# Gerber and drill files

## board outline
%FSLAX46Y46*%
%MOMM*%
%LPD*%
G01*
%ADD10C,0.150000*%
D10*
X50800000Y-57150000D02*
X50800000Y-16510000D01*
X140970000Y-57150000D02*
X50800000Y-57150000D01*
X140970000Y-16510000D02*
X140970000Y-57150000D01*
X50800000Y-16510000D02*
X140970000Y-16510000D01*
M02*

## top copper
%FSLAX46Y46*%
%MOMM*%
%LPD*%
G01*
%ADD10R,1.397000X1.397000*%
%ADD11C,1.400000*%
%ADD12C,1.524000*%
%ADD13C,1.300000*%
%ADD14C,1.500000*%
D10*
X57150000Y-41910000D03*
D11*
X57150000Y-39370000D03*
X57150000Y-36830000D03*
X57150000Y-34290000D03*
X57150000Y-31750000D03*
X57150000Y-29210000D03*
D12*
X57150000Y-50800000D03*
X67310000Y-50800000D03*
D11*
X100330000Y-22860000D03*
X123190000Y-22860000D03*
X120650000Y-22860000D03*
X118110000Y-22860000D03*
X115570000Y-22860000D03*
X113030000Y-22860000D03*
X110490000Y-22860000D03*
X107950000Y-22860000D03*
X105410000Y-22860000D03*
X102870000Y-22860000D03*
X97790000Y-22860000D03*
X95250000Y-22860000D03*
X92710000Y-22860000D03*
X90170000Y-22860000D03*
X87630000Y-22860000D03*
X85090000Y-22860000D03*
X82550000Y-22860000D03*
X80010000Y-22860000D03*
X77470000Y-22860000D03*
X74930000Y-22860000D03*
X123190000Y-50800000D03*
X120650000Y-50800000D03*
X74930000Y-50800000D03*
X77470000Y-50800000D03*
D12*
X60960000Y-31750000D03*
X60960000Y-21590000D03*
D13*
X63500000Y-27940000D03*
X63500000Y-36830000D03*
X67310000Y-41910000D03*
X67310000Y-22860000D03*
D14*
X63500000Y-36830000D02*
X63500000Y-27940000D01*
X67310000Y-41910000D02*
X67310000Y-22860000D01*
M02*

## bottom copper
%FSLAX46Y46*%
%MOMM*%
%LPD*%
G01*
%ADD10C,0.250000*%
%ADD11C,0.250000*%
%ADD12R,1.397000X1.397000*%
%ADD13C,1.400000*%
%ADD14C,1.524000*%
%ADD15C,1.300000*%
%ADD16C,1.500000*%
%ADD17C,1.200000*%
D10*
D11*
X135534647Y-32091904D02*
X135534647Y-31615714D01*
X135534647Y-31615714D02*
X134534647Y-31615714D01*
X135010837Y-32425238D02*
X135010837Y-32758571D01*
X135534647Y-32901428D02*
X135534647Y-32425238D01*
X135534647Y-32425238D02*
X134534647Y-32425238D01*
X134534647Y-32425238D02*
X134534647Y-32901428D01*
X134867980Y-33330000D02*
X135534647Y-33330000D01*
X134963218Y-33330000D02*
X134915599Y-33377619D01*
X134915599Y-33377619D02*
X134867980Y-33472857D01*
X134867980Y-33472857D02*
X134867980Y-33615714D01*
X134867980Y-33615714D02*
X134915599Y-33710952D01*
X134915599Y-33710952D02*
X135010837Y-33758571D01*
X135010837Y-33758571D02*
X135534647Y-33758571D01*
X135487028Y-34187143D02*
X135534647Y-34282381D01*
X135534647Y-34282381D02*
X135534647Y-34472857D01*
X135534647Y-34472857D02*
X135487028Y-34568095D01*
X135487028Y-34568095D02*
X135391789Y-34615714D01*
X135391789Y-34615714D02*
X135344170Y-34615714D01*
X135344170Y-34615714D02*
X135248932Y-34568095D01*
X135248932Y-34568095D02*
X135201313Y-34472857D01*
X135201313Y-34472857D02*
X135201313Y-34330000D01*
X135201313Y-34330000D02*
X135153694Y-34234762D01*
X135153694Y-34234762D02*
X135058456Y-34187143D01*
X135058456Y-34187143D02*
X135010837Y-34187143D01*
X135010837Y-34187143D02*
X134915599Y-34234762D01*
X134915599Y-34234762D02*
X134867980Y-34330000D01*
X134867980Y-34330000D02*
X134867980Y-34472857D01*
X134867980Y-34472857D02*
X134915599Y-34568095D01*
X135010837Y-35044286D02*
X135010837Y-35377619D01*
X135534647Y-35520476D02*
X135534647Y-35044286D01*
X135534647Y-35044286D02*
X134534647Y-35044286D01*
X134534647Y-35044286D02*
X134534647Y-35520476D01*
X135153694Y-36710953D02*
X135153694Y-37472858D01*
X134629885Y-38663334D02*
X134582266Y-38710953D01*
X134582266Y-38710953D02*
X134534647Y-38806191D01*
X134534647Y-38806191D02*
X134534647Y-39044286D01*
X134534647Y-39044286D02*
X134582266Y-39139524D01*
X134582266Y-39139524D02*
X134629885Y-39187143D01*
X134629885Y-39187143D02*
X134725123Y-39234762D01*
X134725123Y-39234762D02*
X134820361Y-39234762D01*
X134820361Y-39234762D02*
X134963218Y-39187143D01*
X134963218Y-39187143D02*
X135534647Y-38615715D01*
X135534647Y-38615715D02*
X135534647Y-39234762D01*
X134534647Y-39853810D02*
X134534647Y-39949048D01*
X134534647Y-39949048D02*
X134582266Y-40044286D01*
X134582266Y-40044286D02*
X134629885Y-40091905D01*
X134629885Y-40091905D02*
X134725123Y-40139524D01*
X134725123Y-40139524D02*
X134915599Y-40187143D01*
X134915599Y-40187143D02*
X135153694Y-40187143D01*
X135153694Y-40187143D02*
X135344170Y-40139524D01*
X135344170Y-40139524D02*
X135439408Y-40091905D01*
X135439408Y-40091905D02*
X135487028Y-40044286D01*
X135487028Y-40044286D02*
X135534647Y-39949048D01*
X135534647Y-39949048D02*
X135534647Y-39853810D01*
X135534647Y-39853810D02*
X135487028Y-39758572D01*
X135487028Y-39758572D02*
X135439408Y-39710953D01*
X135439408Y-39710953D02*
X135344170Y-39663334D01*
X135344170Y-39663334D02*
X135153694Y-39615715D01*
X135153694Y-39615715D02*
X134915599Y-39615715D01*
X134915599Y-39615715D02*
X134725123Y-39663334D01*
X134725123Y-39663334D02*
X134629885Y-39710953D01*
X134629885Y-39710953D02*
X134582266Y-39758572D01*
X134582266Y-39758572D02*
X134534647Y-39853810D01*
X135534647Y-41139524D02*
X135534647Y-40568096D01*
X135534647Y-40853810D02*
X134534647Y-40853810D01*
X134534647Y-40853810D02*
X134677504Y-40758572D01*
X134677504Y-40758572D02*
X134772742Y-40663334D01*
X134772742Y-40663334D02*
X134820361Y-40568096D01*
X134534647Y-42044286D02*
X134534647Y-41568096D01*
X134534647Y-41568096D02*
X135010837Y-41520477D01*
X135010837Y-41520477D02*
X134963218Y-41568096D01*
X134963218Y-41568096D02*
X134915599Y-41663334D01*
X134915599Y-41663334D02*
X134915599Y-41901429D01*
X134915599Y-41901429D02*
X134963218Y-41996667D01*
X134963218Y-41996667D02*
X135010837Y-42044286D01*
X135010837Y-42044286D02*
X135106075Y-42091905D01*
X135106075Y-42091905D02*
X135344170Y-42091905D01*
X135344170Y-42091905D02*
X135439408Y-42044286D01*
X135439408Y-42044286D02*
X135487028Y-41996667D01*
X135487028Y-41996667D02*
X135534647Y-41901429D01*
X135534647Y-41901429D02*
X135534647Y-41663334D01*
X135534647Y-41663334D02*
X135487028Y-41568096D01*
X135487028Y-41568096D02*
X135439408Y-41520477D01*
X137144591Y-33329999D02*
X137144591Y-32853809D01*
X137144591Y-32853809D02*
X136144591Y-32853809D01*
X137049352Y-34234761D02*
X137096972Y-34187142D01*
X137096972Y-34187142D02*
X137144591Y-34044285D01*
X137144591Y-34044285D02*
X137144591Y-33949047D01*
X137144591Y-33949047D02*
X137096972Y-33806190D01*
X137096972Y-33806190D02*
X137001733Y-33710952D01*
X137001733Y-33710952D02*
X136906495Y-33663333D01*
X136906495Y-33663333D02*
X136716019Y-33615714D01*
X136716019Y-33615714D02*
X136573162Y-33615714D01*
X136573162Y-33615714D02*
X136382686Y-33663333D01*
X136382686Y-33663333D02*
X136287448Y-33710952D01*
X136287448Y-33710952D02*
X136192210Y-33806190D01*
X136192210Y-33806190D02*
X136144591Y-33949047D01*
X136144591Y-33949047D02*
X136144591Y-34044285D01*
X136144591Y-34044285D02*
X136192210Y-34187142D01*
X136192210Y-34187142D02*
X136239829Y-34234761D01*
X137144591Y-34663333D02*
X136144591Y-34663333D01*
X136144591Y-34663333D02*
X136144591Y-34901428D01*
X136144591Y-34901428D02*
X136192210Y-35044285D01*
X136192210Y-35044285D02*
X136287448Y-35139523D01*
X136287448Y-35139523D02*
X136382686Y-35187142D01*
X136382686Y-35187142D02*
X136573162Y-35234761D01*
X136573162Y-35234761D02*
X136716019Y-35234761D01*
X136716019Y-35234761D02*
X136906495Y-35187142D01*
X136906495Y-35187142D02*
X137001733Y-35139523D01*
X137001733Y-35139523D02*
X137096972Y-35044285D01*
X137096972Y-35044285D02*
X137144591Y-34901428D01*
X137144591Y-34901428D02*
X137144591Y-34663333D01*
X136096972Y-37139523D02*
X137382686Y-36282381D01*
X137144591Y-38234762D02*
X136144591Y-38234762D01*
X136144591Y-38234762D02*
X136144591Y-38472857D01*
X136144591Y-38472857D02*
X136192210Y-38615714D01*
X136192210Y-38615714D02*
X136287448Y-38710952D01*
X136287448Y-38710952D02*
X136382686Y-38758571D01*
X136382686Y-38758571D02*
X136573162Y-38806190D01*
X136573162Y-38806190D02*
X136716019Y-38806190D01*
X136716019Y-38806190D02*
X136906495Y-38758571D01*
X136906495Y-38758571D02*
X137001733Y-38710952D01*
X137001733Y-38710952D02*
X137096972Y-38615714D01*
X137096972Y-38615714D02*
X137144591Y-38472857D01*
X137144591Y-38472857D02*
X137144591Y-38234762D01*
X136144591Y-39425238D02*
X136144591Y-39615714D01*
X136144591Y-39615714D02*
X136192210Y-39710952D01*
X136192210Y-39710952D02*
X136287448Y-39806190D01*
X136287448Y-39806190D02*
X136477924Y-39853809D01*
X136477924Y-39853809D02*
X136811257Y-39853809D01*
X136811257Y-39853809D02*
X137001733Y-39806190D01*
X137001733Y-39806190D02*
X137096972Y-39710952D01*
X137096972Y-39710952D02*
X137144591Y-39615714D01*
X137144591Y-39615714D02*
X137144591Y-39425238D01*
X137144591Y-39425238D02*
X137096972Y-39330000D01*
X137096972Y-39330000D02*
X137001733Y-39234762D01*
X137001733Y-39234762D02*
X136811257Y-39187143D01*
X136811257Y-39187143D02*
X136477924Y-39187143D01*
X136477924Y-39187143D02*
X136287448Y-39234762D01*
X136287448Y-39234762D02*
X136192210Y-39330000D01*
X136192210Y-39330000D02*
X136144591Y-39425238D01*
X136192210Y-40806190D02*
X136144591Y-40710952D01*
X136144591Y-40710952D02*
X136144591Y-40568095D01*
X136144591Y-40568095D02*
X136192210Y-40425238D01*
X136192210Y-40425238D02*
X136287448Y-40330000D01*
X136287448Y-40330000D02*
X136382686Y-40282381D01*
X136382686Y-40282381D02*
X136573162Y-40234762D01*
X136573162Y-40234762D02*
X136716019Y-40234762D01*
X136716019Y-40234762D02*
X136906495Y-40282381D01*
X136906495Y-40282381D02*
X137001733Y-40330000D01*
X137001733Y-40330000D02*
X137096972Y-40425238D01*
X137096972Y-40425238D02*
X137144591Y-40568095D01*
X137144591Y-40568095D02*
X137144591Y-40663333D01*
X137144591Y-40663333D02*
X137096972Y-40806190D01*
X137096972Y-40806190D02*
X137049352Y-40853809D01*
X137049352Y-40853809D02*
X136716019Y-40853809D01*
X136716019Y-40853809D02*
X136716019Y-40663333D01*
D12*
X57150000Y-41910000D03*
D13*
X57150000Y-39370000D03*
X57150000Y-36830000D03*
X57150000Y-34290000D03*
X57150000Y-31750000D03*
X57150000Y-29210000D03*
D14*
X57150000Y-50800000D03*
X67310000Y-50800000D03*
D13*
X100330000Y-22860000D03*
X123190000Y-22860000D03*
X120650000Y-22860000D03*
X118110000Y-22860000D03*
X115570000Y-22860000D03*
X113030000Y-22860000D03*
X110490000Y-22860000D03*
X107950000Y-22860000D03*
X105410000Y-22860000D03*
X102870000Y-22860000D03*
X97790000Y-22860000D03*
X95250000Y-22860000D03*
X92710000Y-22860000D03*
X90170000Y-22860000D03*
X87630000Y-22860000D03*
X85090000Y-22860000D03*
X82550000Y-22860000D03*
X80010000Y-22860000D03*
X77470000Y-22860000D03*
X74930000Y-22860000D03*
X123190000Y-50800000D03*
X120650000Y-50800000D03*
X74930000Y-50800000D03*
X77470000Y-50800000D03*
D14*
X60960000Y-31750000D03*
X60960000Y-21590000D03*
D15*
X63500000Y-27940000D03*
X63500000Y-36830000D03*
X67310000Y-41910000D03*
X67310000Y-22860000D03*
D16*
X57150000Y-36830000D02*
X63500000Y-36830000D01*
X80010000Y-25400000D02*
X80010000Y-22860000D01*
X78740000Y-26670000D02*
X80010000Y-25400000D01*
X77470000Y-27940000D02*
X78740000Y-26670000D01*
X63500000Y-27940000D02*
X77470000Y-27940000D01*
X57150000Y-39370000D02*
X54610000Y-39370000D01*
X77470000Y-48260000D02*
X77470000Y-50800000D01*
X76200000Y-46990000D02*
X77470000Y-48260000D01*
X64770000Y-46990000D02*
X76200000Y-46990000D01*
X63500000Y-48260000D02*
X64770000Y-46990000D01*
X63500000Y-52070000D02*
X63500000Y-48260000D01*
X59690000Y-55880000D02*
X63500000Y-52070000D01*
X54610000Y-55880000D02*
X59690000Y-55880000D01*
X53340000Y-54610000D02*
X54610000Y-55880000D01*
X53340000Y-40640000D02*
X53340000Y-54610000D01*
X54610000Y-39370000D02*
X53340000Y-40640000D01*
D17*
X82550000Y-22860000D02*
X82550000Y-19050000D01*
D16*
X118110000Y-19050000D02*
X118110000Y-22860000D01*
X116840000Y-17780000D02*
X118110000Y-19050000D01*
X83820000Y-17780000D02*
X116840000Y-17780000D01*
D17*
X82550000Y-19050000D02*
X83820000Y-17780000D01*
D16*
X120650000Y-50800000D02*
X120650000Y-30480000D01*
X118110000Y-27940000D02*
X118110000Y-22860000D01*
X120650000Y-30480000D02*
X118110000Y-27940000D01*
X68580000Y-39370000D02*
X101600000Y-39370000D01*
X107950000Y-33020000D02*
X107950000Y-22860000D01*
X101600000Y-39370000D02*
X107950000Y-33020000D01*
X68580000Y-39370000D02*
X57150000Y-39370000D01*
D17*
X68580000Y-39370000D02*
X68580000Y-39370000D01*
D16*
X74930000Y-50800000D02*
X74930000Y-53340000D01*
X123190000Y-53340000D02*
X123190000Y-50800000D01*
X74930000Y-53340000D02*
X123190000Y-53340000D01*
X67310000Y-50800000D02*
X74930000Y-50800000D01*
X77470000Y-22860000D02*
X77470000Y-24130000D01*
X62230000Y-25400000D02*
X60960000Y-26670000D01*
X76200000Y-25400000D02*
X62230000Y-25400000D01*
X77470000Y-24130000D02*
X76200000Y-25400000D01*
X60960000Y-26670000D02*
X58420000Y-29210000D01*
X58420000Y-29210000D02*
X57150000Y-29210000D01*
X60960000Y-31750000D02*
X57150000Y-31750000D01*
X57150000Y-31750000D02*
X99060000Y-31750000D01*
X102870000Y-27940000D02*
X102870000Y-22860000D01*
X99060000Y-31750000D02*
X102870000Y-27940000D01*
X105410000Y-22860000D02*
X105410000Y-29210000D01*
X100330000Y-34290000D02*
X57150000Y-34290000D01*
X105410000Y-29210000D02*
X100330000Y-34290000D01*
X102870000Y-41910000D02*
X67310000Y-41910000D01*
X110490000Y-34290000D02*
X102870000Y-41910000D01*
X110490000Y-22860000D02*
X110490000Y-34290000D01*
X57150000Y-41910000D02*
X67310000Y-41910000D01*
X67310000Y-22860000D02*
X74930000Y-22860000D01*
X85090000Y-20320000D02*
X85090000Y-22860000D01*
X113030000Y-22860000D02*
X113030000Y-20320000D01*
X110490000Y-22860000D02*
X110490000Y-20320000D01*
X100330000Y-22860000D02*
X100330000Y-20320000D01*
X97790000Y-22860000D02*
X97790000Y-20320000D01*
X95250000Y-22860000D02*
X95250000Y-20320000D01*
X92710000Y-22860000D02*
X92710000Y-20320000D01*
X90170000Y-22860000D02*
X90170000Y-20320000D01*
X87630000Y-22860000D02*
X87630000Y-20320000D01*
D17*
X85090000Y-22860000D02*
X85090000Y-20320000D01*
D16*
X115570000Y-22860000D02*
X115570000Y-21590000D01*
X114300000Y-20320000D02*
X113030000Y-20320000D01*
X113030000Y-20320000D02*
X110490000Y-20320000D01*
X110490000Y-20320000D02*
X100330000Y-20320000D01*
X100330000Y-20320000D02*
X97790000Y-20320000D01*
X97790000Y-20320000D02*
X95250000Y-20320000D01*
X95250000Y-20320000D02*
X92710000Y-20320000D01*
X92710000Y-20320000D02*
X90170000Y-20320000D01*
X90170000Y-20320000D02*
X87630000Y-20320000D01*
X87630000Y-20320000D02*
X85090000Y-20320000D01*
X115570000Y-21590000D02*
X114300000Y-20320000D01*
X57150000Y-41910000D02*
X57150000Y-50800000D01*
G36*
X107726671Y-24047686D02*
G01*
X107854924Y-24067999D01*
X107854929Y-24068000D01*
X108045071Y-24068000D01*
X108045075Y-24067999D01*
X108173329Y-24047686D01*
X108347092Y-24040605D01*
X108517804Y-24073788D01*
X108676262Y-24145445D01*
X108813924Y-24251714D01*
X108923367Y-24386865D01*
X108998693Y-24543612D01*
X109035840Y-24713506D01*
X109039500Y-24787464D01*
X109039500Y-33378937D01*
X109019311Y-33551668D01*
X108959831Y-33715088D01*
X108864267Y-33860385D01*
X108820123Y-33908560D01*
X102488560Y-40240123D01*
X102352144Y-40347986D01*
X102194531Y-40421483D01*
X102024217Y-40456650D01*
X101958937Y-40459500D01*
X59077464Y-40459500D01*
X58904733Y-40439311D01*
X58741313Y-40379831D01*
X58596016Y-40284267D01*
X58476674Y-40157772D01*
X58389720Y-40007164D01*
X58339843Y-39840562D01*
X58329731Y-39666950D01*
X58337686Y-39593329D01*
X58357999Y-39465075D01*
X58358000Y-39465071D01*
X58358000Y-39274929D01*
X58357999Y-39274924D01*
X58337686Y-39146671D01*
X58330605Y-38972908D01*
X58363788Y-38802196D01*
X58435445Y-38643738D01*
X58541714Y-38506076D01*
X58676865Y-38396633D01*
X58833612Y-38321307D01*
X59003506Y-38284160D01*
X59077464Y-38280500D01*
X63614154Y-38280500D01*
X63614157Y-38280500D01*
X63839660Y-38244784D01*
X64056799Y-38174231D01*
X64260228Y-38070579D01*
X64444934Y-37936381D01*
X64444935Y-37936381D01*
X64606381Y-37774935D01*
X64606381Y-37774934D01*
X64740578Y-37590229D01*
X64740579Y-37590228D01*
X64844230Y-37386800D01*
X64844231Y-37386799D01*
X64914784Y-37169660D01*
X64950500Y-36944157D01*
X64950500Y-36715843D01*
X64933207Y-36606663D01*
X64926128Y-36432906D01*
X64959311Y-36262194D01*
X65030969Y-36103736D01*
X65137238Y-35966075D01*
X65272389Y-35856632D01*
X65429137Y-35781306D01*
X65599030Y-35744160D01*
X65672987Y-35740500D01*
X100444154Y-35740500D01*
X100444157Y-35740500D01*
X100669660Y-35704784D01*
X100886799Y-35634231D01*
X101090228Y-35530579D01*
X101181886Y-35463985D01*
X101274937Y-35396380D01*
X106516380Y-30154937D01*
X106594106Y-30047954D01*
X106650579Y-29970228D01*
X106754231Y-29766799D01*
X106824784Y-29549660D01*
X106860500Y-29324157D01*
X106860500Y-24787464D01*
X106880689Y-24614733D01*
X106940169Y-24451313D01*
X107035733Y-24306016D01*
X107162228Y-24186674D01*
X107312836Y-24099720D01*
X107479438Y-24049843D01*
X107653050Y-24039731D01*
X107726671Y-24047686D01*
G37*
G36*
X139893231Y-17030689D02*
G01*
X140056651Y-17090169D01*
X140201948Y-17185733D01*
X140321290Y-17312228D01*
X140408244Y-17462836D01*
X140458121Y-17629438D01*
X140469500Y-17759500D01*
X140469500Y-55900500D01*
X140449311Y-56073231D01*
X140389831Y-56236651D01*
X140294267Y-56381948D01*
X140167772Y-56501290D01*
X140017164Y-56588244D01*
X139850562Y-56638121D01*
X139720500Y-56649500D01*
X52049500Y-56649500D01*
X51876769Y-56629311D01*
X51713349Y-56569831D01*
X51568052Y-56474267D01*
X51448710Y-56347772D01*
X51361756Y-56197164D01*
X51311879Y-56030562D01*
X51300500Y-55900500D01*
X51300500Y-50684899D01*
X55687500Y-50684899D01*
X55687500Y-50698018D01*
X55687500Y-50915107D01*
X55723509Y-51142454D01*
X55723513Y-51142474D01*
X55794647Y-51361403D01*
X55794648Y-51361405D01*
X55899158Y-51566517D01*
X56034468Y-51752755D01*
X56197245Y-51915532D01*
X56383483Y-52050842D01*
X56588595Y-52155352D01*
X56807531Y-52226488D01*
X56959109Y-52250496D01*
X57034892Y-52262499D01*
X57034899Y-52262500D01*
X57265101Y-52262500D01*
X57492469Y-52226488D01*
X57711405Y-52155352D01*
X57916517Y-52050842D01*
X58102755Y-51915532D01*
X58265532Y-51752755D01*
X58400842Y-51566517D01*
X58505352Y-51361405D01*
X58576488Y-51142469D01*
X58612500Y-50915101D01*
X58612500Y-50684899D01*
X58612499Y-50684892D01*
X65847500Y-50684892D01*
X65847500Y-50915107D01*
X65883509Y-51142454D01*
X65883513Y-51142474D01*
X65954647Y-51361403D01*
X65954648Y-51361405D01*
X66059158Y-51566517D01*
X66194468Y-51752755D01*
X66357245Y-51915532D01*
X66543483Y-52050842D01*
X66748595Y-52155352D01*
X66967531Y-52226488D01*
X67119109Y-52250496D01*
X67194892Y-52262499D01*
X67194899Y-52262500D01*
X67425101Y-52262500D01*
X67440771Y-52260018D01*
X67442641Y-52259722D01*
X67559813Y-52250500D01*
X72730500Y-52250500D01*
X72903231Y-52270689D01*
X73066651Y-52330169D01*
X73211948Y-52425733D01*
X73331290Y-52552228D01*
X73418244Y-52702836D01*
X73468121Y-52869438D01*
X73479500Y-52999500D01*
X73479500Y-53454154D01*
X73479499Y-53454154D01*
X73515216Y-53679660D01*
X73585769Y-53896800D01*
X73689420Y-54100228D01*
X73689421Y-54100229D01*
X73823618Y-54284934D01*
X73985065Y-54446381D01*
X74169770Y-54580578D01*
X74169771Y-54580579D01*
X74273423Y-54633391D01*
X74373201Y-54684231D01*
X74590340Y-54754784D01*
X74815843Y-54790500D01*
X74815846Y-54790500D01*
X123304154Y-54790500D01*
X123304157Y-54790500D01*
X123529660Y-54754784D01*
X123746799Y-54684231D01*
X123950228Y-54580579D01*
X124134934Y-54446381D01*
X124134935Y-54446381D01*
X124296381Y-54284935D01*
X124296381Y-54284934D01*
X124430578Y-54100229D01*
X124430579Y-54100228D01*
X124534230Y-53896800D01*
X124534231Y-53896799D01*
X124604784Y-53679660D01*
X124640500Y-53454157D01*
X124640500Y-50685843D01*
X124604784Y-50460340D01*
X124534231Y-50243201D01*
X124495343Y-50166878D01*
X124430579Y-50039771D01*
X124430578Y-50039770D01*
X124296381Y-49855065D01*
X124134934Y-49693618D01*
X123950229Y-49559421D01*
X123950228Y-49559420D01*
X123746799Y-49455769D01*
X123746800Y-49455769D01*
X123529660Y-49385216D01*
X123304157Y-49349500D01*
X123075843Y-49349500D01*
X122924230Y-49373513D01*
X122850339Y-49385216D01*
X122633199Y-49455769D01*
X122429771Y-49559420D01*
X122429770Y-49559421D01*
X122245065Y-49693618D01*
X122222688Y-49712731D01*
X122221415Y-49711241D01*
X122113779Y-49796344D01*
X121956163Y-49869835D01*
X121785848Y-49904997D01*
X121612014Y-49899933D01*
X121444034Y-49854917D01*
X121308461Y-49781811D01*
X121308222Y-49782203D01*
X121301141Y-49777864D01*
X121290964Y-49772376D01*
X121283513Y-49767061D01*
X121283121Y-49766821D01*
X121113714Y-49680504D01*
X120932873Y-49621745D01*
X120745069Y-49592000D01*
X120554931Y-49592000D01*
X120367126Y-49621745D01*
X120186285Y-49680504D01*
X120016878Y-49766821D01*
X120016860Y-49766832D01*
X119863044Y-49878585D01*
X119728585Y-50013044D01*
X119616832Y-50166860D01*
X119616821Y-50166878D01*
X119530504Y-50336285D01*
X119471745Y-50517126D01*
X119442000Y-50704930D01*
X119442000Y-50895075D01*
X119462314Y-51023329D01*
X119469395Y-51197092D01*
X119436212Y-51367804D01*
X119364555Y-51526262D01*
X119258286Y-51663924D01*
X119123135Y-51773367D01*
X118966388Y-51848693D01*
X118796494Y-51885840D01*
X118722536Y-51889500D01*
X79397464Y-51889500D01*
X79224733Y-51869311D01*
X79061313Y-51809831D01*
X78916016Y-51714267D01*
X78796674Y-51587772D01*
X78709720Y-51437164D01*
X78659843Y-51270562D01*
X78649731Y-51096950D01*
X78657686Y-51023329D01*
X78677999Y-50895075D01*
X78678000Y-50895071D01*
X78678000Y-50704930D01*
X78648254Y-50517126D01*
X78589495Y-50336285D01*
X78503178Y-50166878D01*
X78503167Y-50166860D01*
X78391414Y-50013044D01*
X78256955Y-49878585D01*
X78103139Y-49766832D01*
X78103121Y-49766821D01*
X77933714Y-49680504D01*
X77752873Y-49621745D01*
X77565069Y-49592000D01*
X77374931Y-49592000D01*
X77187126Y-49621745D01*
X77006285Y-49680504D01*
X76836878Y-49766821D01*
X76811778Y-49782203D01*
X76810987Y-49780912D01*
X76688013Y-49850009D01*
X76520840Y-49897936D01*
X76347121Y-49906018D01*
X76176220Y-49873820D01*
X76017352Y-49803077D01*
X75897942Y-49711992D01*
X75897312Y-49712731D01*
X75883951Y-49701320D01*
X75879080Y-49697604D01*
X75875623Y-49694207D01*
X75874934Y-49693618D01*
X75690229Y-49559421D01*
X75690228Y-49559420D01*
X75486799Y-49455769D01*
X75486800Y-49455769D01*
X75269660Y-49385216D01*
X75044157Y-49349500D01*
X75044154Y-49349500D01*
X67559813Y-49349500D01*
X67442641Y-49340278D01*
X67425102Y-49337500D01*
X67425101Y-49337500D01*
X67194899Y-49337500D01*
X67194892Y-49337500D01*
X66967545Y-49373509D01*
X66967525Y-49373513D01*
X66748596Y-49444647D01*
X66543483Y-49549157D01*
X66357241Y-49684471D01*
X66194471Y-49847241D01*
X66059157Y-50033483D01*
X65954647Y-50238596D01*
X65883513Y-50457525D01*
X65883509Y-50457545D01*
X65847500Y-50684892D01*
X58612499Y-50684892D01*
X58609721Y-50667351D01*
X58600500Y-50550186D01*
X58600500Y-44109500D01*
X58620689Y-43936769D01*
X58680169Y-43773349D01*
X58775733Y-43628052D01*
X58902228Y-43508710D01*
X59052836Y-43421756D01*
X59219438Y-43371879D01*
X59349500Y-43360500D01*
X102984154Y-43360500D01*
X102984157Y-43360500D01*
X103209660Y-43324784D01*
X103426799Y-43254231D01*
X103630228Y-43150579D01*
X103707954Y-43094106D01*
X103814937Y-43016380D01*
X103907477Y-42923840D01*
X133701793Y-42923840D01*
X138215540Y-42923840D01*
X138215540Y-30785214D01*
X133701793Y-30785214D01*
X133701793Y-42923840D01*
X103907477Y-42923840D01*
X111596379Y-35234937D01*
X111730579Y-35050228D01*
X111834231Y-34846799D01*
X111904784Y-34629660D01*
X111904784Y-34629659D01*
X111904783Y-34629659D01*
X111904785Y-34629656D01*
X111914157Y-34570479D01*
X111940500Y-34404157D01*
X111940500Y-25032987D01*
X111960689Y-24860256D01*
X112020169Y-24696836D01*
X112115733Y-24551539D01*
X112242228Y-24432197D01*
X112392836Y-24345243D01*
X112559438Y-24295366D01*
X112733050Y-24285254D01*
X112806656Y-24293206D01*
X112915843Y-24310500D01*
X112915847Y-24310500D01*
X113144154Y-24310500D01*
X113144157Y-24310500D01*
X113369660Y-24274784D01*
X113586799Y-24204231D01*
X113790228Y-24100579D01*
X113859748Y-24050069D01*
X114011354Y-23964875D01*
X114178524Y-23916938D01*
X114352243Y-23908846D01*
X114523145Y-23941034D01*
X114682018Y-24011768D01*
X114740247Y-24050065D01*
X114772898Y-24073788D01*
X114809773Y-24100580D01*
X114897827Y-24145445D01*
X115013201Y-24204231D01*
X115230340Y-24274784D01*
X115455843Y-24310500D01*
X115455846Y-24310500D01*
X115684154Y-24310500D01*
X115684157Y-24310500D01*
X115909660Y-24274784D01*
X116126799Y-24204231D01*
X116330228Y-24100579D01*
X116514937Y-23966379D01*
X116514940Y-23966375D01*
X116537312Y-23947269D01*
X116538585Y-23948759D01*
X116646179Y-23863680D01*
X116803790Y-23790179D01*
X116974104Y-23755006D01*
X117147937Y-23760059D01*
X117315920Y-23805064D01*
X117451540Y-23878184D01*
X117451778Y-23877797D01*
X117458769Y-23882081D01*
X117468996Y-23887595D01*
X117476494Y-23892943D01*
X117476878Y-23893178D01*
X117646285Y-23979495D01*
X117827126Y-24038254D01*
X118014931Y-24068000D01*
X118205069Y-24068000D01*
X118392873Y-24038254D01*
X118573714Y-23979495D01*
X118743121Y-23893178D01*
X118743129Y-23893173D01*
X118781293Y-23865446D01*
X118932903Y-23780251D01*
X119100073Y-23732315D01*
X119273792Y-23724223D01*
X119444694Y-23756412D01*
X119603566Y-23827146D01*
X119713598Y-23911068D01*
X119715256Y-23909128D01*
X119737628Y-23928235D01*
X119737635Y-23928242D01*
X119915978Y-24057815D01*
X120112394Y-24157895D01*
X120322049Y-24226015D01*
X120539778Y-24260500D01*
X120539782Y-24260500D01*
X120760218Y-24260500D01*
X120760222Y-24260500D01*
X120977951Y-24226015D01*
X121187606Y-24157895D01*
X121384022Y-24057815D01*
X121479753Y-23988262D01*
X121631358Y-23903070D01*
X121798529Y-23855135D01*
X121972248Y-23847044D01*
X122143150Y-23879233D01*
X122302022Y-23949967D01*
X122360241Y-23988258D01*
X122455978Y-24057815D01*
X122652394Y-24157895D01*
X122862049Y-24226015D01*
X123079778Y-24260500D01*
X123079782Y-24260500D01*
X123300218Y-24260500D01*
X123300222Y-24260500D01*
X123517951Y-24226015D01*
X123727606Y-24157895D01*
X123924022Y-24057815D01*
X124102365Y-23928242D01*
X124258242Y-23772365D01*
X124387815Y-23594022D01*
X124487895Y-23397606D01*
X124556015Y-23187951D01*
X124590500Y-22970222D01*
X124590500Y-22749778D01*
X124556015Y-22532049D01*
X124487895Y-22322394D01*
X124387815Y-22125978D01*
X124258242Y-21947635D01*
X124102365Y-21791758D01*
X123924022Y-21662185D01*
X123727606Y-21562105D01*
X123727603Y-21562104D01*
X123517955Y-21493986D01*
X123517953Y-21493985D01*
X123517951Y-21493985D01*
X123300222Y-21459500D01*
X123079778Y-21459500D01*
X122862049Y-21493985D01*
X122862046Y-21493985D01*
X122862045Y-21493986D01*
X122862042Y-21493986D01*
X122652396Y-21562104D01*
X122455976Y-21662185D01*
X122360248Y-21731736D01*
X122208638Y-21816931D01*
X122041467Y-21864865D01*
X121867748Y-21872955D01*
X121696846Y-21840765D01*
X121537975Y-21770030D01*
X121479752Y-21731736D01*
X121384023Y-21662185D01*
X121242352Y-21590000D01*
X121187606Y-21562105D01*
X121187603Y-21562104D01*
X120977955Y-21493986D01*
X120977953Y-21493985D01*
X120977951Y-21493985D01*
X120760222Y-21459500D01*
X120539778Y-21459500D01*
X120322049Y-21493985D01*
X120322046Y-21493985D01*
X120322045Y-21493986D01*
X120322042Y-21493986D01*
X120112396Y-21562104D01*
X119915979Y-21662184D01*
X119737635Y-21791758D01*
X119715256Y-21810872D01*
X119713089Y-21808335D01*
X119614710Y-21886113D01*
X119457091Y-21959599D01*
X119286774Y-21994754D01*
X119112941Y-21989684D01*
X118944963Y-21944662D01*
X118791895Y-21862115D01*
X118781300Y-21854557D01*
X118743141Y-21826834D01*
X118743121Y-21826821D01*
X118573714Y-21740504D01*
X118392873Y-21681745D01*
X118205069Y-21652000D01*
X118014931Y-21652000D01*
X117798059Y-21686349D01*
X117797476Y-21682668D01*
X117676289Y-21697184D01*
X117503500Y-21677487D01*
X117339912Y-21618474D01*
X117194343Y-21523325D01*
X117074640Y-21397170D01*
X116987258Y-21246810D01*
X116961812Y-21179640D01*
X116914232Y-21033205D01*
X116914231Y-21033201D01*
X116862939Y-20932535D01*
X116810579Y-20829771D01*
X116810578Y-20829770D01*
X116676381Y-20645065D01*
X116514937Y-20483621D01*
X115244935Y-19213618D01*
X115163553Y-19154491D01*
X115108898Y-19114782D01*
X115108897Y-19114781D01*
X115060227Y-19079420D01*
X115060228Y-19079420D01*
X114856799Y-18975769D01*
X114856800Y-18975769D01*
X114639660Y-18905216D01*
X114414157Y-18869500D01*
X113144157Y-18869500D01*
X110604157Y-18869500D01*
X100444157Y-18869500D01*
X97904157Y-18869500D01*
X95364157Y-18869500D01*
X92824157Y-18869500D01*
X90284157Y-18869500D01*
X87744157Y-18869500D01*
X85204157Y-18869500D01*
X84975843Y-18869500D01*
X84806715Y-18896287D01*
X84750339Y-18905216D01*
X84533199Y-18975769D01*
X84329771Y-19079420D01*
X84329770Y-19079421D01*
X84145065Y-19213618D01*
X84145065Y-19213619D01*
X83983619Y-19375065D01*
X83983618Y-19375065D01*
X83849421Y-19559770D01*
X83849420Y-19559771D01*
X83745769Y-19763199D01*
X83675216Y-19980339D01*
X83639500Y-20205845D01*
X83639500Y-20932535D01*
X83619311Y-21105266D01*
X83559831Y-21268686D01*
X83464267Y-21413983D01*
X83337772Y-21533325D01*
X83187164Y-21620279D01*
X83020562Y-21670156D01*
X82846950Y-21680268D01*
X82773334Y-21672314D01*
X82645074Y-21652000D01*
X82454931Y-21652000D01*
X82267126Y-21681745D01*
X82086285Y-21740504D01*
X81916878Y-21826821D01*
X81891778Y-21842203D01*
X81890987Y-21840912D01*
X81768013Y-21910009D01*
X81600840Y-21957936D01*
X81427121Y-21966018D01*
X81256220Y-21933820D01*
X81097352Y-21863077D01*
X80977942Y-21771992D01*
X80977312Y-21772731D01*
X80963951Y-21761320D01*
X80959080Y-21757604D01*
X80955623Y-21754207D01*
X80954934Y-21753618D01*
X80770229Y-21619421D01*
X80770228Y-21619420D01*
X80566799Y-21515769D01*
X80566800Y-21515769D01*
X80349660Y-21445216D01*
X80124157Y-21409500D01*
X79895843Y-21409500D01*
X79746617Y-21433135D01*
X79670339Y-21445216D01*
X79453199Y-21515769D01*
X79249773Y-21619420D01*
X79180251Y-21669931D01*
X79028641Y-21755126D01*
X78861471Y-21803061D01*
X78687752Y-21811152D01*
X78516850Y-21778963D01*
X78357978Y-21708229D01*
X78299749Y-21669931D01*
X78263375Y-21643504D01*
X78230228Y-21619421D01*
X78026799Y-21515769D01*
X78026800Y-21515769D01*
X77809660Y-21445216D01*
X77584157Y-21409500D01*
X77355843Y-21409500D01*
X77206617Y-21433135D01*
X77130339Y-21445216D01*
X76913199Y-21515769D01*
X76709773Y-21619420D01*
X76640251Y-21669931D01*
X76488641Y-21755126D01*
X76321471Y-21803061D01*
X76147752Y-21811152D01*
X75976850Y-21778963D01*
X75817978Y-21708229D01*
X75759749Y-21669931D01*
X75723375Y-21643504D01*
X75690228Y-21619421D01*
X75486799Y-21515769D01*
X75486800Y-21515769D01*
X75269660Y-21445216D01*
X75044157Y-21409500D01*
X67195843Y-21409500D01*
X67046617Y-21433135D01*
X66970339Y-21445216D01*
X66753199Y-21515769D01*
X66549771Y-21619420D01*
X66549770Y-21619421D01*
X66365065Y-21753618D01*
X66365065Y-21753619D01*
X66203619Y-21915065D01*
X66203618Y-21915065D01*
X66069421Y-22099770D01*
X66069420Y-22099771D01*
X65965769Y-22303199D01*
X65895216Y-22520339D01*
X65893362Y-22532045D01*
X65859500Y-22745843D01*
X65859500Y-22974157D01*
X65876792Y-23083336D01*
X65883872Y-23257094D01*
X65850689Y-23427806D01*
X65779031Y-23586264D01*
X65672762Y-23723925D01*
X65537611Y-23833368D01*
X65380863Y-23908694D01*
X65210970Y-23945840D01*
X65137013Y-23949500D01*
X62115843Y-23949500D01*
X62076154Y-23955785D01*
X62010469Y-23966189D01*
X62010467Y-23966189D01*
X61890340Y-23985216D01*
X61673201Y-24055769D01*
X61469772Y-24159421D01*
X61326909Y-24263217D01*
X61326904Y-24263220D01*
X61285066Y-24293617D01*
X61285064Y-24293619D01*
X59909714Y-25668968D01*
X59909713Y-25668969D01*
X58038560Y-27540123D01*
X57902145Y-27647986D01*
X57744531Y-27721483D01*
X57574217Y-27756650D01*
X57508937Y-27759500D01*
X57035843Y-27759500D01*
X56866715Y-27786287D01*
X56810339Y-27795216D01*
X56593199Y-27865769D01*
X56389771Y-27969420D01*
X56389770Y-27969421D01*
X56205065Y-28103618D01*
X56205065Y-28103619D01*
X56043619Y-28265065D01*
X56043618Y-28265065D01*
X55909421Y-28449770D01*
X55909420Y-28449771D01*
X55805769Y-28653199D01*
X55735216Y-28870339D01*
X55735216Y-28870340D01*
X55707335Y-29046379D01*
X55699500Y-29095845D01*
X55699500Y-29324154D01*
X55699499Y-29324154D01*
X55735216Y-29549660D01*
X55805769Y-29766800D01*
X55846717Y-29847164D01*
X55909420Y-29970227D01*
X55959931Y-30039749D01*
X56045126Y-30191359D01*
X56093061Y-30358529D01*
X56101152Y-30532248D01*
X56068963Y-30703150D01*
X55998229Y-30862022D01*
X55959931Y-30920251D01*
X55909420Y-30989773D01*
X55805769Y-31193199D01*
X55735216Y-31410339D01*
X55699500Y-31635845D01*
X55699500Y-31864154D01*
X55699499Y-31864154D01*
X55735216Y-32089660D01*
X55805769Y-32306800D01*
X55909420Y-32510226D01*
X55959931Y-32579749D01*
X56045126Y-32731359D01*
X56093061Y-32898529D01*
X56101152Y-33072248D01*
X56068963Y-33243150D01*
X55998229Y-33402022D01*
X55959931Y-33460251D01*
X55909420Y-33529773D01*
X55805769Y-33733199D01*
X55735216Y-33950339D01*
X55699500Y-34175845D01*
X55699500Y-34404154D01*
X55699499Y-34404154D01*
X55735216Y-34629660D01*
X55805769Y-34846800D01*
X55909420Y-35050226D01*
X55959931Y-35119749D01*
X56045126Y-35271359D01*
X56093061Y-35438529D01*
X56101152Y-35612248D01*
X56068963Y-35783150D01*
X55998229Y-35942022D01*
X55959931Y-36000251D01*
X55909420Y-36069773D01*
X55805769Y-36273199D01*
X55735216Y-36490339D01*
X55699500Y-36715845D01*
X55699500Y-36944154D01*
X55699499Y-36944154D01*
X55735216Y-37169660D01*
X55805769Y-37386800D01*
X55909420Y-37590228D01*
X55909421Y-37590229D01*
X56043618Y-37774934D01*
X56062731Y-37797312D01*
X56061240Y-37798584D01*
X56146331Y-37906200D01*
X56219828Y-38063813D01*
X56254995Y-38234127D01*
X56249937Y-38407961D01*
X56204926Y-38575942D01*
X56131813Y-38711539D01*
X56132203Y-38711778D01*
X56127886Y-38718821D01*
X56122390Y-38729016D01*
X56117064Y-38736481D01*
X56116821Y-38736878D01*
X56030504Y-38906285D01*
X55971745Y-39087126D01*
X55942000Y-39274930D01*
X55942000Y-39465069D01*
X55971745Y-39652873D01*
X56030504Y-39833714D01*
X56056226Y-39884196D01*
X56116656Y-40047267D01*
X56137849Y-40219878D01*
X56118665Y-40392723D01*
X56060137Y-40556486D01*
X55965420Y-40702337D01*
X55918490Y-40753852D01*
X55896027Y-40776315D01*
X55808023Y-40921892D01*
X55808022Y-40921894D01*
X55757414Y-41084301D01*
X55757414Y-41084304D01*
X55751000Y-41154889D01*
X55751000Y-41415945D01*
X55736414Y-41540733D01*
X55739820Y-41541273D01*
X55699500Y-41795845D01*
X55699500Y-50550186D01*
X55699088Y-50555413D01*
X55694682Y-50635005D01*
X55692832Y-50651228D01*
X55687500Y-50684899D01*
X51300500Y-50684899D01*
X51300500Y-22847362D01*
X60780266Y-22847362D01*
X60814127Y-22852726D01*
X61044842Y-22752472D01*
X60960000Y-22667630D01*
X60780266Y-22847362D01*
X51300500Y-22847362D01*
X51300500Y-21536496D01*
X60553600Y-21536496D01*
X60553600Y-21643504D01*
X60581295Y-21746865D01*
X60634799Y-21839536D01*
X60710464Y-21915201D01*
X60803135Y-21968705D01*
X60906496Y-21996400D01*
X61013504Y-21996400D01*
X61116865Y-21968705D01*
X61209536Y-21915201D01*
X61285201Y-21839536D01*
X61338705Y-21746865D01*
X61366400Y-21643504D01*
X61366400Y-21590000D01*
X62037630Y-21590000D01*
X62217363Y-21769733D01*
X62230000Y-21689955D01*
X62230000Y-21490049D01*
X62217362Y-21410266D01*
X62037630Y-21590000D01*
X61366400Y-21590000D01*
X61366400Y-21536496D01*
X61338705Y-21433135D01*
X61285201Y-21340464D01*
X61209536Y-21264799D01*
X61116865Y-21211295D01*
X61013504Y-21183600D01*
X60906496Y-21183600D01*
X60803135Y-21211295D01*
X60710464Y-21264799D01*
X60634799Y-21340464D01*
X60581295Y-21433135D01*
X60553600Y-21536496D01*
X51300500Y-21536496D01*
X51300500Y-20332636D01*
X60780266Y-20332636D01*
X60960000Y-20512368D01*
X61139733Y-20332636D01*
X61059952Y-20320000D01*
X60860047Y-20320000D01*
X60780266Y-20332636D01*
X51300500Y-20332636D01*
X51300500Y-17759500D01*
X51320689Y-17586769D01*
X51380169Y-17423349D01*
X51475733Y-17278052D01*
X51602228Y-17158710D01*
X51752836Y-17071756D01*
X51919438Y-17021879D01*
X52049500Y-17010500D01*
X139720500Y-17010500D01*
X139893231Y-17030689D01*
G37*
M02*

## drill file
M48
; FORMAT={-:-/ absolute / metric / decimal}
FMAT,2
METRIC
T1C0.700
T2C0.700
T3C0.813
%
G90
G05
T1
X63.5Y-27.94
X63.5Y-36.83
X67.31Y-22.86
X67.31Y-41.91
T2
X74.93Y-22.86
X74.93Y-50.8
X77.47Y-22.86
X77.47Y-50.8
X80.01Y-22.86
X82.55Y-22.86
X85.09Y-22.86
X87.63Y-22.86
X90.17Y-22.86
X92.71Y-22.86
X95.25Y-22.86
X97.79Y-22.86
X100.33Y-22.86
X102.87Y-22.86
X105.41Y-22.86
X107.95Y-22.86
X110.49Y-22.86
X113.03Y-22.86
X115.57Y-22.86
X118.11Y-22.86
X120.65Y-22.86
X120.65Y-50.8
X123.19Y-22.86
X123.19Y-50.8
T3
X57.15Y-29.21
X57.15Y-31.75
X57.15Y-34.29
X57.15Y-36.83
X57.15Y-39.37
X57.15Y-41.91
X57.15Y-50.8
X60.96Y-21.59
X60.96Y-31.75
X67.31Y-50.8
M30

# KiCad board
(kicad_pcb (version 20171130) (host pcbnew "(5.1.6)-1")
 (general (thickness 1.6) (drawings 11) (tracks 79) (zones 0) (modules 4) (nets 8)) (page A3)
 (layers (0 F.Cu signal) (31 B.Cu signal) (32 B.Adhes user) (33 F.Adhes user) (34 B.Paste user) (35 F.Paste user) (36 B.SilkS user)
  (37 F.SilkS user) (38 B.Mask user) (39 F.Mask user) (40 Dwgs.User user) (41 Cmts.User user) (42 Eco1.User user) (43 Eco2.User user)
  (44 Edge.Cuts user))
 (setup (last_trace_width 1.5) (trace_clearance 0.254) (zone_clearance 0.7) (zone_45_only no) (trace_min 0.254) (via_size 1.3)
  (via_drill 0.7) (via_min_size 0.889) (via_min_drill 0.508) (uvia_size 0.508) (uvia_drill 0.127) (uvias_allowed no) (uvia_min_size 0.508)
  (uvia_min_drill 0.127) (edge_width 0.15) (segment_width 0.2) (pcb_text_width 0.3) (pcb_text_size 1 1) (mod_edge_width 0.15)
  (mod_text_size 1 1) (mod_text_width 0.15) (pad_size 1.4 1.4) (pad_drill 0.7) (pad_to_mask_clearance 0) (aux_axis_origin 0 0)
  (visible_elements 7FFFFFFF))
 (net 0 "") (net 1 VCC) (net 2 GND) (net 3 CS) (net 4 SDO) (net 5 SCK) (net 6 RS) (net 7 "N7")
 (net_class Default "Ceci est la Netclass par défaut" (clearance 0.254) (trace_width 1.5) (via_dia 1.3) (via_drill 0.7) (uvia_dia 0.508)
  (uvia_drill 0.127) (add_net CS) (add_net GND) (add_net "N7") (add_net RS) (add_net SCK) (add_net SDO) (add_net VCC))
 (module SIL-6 (layer F.Cu) (at 57.15 35.56 90)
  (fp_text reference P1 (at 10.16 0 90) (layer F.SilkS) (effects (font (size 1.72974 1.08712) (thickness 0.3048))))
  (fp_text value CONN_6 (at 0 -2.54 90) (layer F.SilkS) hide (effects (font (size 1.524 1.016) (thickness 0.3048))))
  (pad 1 thru_hole rect (at -6.35 0 90) (size 1.397 1.397) (drill 0.8128) (layers *.Cu *.Mask F.SilkS) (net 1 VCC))
  (pad 2 thru_hole circle (at -3.81 0 90) (size 1.4 1.4) (drill 0.8128) (layers *.Cu *.Mask F.SilkS) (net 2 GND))
  (pad 3 thru_hole circle (at -1.27 0 90) (size 1.4 1.4) (drill 0.8128) (layers *.Cu *.Mask F.SilkS) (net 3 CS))
  (pad 4 thru_hole circle (at 1.27 0 90) (size 1.4 1.4) (drill 0.8128) (layers *.Cu *.Mask F.SilkS) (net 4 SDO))
  (pad 5 thru_hole circle (at 3.81 0 90) (size 1.4 1.4) (drill 0.8128) (layers *.Cu *.Mask F.SilkS) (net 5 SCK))
  (pad 6 thru_hole circle (at 6.35 0 90) (size 1.4 1.4) (drill 0.8128) (layers *.Cu *.Mask F.SilkS) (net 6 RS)))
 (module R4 (layer F.Cu) (at 62.23 50.8) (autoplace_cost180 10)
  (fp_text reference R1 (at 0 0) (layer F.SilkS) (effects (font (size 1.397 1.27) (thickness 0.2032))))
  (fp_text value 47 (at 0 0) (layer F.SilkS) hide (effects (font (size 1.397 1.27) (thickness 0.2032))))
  (pad 1 thru_hole circle (at -5.08 0) (size 1.524 1.524) (drill 0.8128) (layers *.Cu *.Mask F.SilkS) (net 1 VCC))
  (pad 2 thru_hole circle (at 5.08 0) (size 1.524 1.524) (drill 0.8128) (layers *.Cu *.Mask F.SilkS) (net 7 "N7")))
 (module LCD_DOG (layer F.Cu) (at 123.19 22.86)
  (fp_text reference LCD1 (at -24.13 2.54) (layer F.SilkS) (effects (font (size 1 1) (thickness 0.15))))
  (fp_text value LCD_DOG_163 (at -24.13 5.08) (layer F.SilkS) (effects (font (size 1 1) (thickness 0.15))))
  (pad 30 thru_hole circle (at -22.86 0) (size 1.4 1.4) (drill 0.7) (layers *.Cu *.Mask F.SilkS) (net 1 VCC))
  (pad 21 thru_hole circle (at 0 0) (size 1.4 1.4) (drill 0.7) (layers *.Cu *.Mask F.SilkS))
  (pad 22 thru_hole circle (at -2.54 0) (size 1.4 1.4) (drill 0.7) (layers *.Cu *.Mask F.SilkS))
  (pad 23 thru_hole circle (at -5.08 0) (size 1.4 1.4) (drill 0.7) (layers *.Cu *.Mask F.SilkS) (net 2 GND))
  (pad 24 thru_hole circle (at -7.62 0) (size 1.4 1.4) (drill 0.7) (layers *.Cu *.Mask F.SilkS) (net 1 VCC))
  (pad 25 thru_hole circle (at -10.16 0) (size 1.4 1.4) (drill 0.7) (layers *.Cu *.Mask F.SilkS) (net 1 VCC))
  (pad 26 thru_hole circle (at -12.7 0) (size 1.4 1.4) (drill 0.7) (layers *.Cu *.Mask F.SilkS) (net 1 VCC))
  (pad 27 thru_hole circle (at -15.24 0) (size 1.4 1.4) (drill 0.7) (layers *.Cu *.Mask F.SilkS) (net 2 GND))
  (pad 28 thru_hole circle (at -17.78 0) (size 1.4 1.4) (drill 0.7) (layers *.Cu *.Mask F.SilkS) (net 4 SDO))
  (pad 29 thru_hole circle (at -20.32 0) (size 1.4 1.4) (drill 0.7) (layers *.Cu *.Mask F.SilkS) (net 5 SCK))
  (pad 31 thru_hole circle (at -25.4 0) (size 1.4 1.4) (drill 0.7) (layers *.Cu *.Mask F.SilkS) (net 1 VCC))
  (pad 32 thru_hole circle (at -27.94 0) (size 1.4 1.4) (drill 0.7) (layers *.Cu *.Mask F.SilkS) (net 1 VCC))
  (pad 33 thru_hole circle (at -30.48 0) (size 1.4 1.4) (drill 0.7) (layers *.Cu *.Mask F.SilkS) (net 1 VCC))
  (pad 34 thru_hole circle (at -33.02 0) (size 1.4 1.4) (drill 0.7) (layers *.Cu *.Mask F.SilkS) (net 1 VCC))
  (pad 35 thru_hole circle (at -35.56 0) (size 1.4 1.4) (drill 0.7) (layers *.Cu *.Mask F.SilkS) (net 1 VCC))
  (pad 36 thru_hole circle (at -38.1 0) (size 1.4 1.4) (drill 0.7) (layers *.Cu *.Mask F.SilkS) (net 1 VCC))
  (pad 37 thru_hole circle (at -40.64 0) (size 1.4 1.4) (drill 0.7) (layers *.Cu *.Mask F.SilkS) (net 2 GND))
  (pad 38 thru_hole circle (at -43.18 0) (size 1.4 1.4) (drill 0.7) (layers *.Cu *.Mask F.SilkS) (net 3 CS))
  (pad 39 thru_hole circle (at -45.72 0) (size 1.4 1.4) (drill 0.7) (layers *.Cu *.Mask F.SilkS) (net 6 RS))
  (pad 40 thru_hole circle (at -48.26 0) (size 1.4 1.4) (drill 0.7) (layers *.Cu *.Mask F.SilkS) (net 1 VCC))
  (pad 20 thru_hole circle (at 0 27.94) (size 1.4 1.4) (drill 0.7) (layers *.Cu *.Mask F.SilkS) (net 7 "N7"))
  (pad 19 thru_hole circle (at -2.54 27.94) (size 1.4 1.4) (drill 0.7) (layers *.Cu *.Mask F.SilkS) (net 2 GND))
  (pad 1 thru_hole circle (at -48.26 27.94) (size 1.4 1.4) (drill 0.7) (layers *.Cu *.Mask F.SilkS) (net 7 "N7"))
  (pad 2 thru_hole circle (at -45.72 27.94) (size 1.4 1.4) (drill 0.7) (layers *.Cu *.Mask F.SilkS) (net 2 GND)))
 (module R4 (layer F.Cu) (at 60.96 26.67 90) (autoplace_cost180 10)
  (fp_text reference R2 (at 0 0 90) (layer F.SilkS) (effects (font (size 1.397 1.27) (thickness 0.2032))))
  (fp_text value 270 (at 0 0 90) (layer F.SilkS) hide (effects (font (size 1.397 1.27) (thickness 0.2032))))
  (pad 1 thru_hole circle (at -5.08 0 90) (size 1.524 1.524) (drill 0.8128) (layers *.Cu *.Mask F.SilkS) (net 5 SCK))
  (pad 2 thru_hole circle (at 5.08 0 90) (size 1.524 1.524) (drill 0.8128) (layers *.Cu *.Mask F.SilkS) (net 2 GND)))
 (gr_line (start 50.8 57.15) (end 50.8 16.51) (layer Edge.Cuts) (width 0.15))
 (gr_line (start 140.97 57.15) (end 50.8 57.15) (layer Edge.Cuts) (width 0.15))
 (gr_line (start 140.97 16.51) (end 140.97 57.15) (layer Edge.Cuts) (width 0.15))
 (gr_line (start 50.8 16.51) (end 140.97 16.51) (layer Edge.Cuts) (width 0.15))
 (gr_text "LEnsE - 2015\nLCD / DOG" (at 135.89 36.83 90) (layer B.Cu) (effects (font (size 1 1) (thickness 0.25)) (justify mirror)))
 (segment (start 57.15 36.83) (end 63.5 36.83) (width 1.5) (layer B.Cu) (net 3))
 (segment (start 80.01 25.4) (end 80.01 22.86) (width 1.5) (layer B.Cu) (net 3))
 (segment (start 78.74 26.67) (end 80.01 25.4) (width 1.5) (layer B.Cu) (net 3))
 (segment (start 77.47 27.94) (end 78.74 26.67) (width 1.5) (layer B.Cu) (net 3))
 (segment (start 63.5 27.94) (end 77.47 27.94) (width 1.5) (layer B.Cu) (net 3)) (via (at 63.5 27.94) (size 1.3) (layers F.Cu B.Cu) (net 3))
 (segment (start 63.5 36.83) (end 63.5 27.94) (width 1.5) (layer F.Cu) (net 3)) (via (at 63.5 36.83) (size 1.3) (layers F.Cu B.Cu) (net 3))
 (segment (start 57.15 39.37) (end 54.61 39.37) (width 1.5) (layer B.Cu) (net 2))
 (segment (start 77.47 48.26) (end 77.47 50.8) (width 1.5) (layer B.Cu) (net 2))
 (segment (start 76.2 46.99) (end 77.47 48.26) (width 1.5) (layer B.Cu) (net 2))
 (segment (start 64.77 46.99) (end 76.2 46.99) (width 1.5) (layer B.Cu) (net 2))
 (segment (start 63.5 48.26) (end 64.77 46.99) (width 1.5) (layer B.Cu) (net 2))
 (segment (start 63.5 52.07) (end 63.5 48.26) (width 1.5) (layer B.Cu) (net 2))
 (segment (start 59.69 55.88) (end 63.5 52.07) (width 1.5) (layer B.Cu) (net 2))
 (segment (start 54.61 55.88) (end 59.69 55.88) (width 1.5) (layer B.Cu) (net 2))
 (segment (start 53.34 54.61) (end 54.61 55.88) (width 1.5) (layer B.Cu) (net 2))
 (segment (start 53.34 40.64) (end 53.34 54.61) (width 1.5) (layer B.Cu) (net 2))
 (segment (start 54.61 39.37) (end 53.34 40.64) (width 1.5) (layer B.Cu) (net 2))
 (segment (start 82.55 22.86) (end 82.55 19.05) (width 1.2) (layer B.Cu) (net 2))
 (segment (start 118.11 19.05) (end 118.11 22.86) (width 1.5) (layer B.Cu) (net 2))
 (segment (start 116.84 17.78) (end 118.11 19.05) (width 1.5) (layer B.Cu) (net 2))
 (segment (start 83.82 17.78) (end 116.84 17.78) (width 1.5) (layer B.Cu) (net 2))
 (segment (start 82.55 19.05) (end 83.82 17.78) (width 1.2) (layer B.Cu) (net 2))
 (segment (start 120.65 50.8) (end 120.65 30.48) (width 1.5) (layer B.Cu) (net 2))
 (segment (start 118.11 27.94) (end 118.11 22.86) (width 1.5) (layer B.Cu) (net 2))
 (segment (start 120.65 30.48) (end 118.11 27.94) (width 1.5) (layer B.Cu) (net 2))
 (segment (start 68.58 39.37) (end 101.6 39.37) (width 1.5) (layer B.Cu) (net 2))
 (segment (start 107.95 33.02) (end 107.95 22.86) (width 1.5) (layer B.Cu) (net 2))
 (segment (start 101.6 39.37) (end 107.95 33.02) (width 1.5) (layer B.Cu) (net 2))
 (segment (start 68.58 39.37) (end 57.15 39.37) (width 1.5) (layer B.Cu) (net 2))
 (segment (start 68.58 39.37) (end 68.58 39.37) (width 1.2) (layer B.Cu) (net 2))
 (segment (start 74.93 50.8) (end 74.93 53.34) (width 1.5) (layer B.Cu) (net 7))
 (segment (start 123.19 53.34) (end 123.19 50.8) (width 1.5) (layer B.Cu) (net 7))
 (segment (start 74.93 53.34) (end 123.19 53.34) (width 1.5) (layer B.Cu) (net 7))
 (segment (start 67.31 50.8) (end 74.93 50.8) (width 1.5) (layer B.Cu) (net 7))
 (segment (start 77.47 22.86) (end 77.47 24.13) (width 1.5) (layer B.Cu) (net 6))
 (segment (start 62.23 25.4) (end 60.96 26.67) (width 1.5) (layer B.Cu) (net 6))
 (segment (start 76.2 25.4) (end 62.23 25.4) (width 1.5) (layer B.Cu) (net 6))
 (segment (start 77.47 24.13) (end 76.2 25.4) (width 1.5) (layer B.Cu) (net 6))
 (segment (start 60.96 26.67) (end 58.42 29.21) (width 1.5) (layer B.Cu) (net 6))
 (segment (start 58.42 29.21) (end 57.15 29.21) (width 1.5) (layer B.Cu) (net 6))
 (segment (start 60.96 31.75) (end 57.15 31.75) (width 1.5) (layer B.Cu) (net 5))
 (segment (start 57.15 31.75) (end 99.06 31.75) (width 1.5) (layer B.Cu) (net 5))
 (segment (start 102.87 27.94) (end 102.87 22.86) (width 1.5) (layer B.Cu) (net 5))
 (segment (start 99.06 31.75) (end 102.87 27.94) (width 1.5) (layer B.Cu) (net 5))
 (segment (start 105.41 22.86) (end 105.41 29.21) (width 1.5) (layer B.Cu) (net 4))
 (segment (start 100.33 34.29) (end 57.15 34.29) (width 1.5) (layer B.Cu) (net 4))
 (segment (start 105.41 29.21) (end 100.33 34.29) (width 1.5) (layer B.Cu) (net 4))
 (segment (start 102.87 41.91) (end 67.31 41.91) (width 1.5) (layer B.Cu) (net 1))
 (segment (start 110.49 34.29) (end 102.87 41.91) (width 1.5) (layer B.Cu) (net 1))
 (segment (start 110.49 22.86) (end 110.49 34.29) (width 1.5) (layer B.Cu) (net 1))
 (segment (start 57.15 41.91) (end 67.31 41.91) (width 1.5) (layer B.Cu) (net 1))
 (segment (start 67.31 22.86) (end 74.93 22.86) (width 1.5) (layer B.Cu) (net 1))
 (via (at 67.31 41.91) (size 1.3) (layers F.Cu B.Cu) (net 1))
 (segment (start 67.31 41.91) (end 67.31 22.86) (width 1.5) (layer F.Cu) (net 1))
 (via (at 67.31 22.86) (size 1.3) (layers F.Cu B.Cu) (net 1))
 (segment (start 85.09 20.32) (end 85.09 22.86) (width 1.5) (layer B.Cu) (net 1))
 (segment (start 113.03 22.86) (end 113.03 20.32) (width 1.5) (layer B.Cu) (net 1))
 (segment (start 110.49 22.86) (end 110.49 20.32) (width 1.5) (layer B.Cu) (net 1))
 (segment (start 100.33 22.86) (end 100.33 20.32) (width 1.5) (layer B.Cu) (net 1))
 (segment (start 97.79 22.86) (end 97.79 20.32) (width 1.5) (layer B.Cu) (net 1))
 (segment (start 95.25 22.86) (end 95.25 20.32) (width 1.5) (layer B.Cu) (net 1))
 (segment (start 92.71 22.86) (end 92.71 20.32) (width 1.5) (layer B.Cu) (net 1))
 (segment (start 90.17 22.86) (end 90.17 20.32) (width 1.5) (layer B.Cu) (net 1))
 (segment (start 87.63 22.86) (end 87.63 20.32) (width 1.5) (layer B.Cu) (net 1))
 (segment (start 85.09 22.86) (end 85.09 20.32) (width 1.2) (layer B.Cu) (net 1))
 (segment (start 115.57 22.86) (end 115.57 21.59) (width 1.5) (layer B.Cu) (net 1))
 (segment (start 114.3 20.32) (end 113.03 20.32) (width 1.5) (layer B.Cu) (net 1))
 (segment (start 113.03 20.32) (end 110.49 20.32) (width 1.5) (layer B.Cu) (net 1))
 (segment (start 110.49 20.32) (end 100.33 20.32) (width 1.5) (layer B.Cu) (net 1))
 (segment (start 100.33 20.32) (end 97.79 20.32) (width 1.5) (layer B.Cu) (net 1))
 (segment (start 97.79 20.32) (end 95.25 20.32) (width 1.5) (layer B.Cu) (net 1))
 (segment (start 95.25 20.32) (end 92.71 20.32) (width 1.5) (layer B.Cu) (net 1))
 (segment (start 92.71 20.32) (end 90.17 20.32) (width 1.5) (layer B.Cu) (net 1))
 (segment (start 90.17 20.32) (end 87.63 20.32) (width 1.5) (layer B.Cu) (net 1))
 (segment (start 87.63 20.32) (end 85.09 20.32) (width 1.5) (layer B.Cu) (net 1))
 (segment (start 115.57 21.59) (end 114.3 20.32) (width 1.5) (layer B.Cu) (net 1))
 (segment (start 57.15 41.91) (end 57.15 50.8) (width 1.5) (layer B.Cu) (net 1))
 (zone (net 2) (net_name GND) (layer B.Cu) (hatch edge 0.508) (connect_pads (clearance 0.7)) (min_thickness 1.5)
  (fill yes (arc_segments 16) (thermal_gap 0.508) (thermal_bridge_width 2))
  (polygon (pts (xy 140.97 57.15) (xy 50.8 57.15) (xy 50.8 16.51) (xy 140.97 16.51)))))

